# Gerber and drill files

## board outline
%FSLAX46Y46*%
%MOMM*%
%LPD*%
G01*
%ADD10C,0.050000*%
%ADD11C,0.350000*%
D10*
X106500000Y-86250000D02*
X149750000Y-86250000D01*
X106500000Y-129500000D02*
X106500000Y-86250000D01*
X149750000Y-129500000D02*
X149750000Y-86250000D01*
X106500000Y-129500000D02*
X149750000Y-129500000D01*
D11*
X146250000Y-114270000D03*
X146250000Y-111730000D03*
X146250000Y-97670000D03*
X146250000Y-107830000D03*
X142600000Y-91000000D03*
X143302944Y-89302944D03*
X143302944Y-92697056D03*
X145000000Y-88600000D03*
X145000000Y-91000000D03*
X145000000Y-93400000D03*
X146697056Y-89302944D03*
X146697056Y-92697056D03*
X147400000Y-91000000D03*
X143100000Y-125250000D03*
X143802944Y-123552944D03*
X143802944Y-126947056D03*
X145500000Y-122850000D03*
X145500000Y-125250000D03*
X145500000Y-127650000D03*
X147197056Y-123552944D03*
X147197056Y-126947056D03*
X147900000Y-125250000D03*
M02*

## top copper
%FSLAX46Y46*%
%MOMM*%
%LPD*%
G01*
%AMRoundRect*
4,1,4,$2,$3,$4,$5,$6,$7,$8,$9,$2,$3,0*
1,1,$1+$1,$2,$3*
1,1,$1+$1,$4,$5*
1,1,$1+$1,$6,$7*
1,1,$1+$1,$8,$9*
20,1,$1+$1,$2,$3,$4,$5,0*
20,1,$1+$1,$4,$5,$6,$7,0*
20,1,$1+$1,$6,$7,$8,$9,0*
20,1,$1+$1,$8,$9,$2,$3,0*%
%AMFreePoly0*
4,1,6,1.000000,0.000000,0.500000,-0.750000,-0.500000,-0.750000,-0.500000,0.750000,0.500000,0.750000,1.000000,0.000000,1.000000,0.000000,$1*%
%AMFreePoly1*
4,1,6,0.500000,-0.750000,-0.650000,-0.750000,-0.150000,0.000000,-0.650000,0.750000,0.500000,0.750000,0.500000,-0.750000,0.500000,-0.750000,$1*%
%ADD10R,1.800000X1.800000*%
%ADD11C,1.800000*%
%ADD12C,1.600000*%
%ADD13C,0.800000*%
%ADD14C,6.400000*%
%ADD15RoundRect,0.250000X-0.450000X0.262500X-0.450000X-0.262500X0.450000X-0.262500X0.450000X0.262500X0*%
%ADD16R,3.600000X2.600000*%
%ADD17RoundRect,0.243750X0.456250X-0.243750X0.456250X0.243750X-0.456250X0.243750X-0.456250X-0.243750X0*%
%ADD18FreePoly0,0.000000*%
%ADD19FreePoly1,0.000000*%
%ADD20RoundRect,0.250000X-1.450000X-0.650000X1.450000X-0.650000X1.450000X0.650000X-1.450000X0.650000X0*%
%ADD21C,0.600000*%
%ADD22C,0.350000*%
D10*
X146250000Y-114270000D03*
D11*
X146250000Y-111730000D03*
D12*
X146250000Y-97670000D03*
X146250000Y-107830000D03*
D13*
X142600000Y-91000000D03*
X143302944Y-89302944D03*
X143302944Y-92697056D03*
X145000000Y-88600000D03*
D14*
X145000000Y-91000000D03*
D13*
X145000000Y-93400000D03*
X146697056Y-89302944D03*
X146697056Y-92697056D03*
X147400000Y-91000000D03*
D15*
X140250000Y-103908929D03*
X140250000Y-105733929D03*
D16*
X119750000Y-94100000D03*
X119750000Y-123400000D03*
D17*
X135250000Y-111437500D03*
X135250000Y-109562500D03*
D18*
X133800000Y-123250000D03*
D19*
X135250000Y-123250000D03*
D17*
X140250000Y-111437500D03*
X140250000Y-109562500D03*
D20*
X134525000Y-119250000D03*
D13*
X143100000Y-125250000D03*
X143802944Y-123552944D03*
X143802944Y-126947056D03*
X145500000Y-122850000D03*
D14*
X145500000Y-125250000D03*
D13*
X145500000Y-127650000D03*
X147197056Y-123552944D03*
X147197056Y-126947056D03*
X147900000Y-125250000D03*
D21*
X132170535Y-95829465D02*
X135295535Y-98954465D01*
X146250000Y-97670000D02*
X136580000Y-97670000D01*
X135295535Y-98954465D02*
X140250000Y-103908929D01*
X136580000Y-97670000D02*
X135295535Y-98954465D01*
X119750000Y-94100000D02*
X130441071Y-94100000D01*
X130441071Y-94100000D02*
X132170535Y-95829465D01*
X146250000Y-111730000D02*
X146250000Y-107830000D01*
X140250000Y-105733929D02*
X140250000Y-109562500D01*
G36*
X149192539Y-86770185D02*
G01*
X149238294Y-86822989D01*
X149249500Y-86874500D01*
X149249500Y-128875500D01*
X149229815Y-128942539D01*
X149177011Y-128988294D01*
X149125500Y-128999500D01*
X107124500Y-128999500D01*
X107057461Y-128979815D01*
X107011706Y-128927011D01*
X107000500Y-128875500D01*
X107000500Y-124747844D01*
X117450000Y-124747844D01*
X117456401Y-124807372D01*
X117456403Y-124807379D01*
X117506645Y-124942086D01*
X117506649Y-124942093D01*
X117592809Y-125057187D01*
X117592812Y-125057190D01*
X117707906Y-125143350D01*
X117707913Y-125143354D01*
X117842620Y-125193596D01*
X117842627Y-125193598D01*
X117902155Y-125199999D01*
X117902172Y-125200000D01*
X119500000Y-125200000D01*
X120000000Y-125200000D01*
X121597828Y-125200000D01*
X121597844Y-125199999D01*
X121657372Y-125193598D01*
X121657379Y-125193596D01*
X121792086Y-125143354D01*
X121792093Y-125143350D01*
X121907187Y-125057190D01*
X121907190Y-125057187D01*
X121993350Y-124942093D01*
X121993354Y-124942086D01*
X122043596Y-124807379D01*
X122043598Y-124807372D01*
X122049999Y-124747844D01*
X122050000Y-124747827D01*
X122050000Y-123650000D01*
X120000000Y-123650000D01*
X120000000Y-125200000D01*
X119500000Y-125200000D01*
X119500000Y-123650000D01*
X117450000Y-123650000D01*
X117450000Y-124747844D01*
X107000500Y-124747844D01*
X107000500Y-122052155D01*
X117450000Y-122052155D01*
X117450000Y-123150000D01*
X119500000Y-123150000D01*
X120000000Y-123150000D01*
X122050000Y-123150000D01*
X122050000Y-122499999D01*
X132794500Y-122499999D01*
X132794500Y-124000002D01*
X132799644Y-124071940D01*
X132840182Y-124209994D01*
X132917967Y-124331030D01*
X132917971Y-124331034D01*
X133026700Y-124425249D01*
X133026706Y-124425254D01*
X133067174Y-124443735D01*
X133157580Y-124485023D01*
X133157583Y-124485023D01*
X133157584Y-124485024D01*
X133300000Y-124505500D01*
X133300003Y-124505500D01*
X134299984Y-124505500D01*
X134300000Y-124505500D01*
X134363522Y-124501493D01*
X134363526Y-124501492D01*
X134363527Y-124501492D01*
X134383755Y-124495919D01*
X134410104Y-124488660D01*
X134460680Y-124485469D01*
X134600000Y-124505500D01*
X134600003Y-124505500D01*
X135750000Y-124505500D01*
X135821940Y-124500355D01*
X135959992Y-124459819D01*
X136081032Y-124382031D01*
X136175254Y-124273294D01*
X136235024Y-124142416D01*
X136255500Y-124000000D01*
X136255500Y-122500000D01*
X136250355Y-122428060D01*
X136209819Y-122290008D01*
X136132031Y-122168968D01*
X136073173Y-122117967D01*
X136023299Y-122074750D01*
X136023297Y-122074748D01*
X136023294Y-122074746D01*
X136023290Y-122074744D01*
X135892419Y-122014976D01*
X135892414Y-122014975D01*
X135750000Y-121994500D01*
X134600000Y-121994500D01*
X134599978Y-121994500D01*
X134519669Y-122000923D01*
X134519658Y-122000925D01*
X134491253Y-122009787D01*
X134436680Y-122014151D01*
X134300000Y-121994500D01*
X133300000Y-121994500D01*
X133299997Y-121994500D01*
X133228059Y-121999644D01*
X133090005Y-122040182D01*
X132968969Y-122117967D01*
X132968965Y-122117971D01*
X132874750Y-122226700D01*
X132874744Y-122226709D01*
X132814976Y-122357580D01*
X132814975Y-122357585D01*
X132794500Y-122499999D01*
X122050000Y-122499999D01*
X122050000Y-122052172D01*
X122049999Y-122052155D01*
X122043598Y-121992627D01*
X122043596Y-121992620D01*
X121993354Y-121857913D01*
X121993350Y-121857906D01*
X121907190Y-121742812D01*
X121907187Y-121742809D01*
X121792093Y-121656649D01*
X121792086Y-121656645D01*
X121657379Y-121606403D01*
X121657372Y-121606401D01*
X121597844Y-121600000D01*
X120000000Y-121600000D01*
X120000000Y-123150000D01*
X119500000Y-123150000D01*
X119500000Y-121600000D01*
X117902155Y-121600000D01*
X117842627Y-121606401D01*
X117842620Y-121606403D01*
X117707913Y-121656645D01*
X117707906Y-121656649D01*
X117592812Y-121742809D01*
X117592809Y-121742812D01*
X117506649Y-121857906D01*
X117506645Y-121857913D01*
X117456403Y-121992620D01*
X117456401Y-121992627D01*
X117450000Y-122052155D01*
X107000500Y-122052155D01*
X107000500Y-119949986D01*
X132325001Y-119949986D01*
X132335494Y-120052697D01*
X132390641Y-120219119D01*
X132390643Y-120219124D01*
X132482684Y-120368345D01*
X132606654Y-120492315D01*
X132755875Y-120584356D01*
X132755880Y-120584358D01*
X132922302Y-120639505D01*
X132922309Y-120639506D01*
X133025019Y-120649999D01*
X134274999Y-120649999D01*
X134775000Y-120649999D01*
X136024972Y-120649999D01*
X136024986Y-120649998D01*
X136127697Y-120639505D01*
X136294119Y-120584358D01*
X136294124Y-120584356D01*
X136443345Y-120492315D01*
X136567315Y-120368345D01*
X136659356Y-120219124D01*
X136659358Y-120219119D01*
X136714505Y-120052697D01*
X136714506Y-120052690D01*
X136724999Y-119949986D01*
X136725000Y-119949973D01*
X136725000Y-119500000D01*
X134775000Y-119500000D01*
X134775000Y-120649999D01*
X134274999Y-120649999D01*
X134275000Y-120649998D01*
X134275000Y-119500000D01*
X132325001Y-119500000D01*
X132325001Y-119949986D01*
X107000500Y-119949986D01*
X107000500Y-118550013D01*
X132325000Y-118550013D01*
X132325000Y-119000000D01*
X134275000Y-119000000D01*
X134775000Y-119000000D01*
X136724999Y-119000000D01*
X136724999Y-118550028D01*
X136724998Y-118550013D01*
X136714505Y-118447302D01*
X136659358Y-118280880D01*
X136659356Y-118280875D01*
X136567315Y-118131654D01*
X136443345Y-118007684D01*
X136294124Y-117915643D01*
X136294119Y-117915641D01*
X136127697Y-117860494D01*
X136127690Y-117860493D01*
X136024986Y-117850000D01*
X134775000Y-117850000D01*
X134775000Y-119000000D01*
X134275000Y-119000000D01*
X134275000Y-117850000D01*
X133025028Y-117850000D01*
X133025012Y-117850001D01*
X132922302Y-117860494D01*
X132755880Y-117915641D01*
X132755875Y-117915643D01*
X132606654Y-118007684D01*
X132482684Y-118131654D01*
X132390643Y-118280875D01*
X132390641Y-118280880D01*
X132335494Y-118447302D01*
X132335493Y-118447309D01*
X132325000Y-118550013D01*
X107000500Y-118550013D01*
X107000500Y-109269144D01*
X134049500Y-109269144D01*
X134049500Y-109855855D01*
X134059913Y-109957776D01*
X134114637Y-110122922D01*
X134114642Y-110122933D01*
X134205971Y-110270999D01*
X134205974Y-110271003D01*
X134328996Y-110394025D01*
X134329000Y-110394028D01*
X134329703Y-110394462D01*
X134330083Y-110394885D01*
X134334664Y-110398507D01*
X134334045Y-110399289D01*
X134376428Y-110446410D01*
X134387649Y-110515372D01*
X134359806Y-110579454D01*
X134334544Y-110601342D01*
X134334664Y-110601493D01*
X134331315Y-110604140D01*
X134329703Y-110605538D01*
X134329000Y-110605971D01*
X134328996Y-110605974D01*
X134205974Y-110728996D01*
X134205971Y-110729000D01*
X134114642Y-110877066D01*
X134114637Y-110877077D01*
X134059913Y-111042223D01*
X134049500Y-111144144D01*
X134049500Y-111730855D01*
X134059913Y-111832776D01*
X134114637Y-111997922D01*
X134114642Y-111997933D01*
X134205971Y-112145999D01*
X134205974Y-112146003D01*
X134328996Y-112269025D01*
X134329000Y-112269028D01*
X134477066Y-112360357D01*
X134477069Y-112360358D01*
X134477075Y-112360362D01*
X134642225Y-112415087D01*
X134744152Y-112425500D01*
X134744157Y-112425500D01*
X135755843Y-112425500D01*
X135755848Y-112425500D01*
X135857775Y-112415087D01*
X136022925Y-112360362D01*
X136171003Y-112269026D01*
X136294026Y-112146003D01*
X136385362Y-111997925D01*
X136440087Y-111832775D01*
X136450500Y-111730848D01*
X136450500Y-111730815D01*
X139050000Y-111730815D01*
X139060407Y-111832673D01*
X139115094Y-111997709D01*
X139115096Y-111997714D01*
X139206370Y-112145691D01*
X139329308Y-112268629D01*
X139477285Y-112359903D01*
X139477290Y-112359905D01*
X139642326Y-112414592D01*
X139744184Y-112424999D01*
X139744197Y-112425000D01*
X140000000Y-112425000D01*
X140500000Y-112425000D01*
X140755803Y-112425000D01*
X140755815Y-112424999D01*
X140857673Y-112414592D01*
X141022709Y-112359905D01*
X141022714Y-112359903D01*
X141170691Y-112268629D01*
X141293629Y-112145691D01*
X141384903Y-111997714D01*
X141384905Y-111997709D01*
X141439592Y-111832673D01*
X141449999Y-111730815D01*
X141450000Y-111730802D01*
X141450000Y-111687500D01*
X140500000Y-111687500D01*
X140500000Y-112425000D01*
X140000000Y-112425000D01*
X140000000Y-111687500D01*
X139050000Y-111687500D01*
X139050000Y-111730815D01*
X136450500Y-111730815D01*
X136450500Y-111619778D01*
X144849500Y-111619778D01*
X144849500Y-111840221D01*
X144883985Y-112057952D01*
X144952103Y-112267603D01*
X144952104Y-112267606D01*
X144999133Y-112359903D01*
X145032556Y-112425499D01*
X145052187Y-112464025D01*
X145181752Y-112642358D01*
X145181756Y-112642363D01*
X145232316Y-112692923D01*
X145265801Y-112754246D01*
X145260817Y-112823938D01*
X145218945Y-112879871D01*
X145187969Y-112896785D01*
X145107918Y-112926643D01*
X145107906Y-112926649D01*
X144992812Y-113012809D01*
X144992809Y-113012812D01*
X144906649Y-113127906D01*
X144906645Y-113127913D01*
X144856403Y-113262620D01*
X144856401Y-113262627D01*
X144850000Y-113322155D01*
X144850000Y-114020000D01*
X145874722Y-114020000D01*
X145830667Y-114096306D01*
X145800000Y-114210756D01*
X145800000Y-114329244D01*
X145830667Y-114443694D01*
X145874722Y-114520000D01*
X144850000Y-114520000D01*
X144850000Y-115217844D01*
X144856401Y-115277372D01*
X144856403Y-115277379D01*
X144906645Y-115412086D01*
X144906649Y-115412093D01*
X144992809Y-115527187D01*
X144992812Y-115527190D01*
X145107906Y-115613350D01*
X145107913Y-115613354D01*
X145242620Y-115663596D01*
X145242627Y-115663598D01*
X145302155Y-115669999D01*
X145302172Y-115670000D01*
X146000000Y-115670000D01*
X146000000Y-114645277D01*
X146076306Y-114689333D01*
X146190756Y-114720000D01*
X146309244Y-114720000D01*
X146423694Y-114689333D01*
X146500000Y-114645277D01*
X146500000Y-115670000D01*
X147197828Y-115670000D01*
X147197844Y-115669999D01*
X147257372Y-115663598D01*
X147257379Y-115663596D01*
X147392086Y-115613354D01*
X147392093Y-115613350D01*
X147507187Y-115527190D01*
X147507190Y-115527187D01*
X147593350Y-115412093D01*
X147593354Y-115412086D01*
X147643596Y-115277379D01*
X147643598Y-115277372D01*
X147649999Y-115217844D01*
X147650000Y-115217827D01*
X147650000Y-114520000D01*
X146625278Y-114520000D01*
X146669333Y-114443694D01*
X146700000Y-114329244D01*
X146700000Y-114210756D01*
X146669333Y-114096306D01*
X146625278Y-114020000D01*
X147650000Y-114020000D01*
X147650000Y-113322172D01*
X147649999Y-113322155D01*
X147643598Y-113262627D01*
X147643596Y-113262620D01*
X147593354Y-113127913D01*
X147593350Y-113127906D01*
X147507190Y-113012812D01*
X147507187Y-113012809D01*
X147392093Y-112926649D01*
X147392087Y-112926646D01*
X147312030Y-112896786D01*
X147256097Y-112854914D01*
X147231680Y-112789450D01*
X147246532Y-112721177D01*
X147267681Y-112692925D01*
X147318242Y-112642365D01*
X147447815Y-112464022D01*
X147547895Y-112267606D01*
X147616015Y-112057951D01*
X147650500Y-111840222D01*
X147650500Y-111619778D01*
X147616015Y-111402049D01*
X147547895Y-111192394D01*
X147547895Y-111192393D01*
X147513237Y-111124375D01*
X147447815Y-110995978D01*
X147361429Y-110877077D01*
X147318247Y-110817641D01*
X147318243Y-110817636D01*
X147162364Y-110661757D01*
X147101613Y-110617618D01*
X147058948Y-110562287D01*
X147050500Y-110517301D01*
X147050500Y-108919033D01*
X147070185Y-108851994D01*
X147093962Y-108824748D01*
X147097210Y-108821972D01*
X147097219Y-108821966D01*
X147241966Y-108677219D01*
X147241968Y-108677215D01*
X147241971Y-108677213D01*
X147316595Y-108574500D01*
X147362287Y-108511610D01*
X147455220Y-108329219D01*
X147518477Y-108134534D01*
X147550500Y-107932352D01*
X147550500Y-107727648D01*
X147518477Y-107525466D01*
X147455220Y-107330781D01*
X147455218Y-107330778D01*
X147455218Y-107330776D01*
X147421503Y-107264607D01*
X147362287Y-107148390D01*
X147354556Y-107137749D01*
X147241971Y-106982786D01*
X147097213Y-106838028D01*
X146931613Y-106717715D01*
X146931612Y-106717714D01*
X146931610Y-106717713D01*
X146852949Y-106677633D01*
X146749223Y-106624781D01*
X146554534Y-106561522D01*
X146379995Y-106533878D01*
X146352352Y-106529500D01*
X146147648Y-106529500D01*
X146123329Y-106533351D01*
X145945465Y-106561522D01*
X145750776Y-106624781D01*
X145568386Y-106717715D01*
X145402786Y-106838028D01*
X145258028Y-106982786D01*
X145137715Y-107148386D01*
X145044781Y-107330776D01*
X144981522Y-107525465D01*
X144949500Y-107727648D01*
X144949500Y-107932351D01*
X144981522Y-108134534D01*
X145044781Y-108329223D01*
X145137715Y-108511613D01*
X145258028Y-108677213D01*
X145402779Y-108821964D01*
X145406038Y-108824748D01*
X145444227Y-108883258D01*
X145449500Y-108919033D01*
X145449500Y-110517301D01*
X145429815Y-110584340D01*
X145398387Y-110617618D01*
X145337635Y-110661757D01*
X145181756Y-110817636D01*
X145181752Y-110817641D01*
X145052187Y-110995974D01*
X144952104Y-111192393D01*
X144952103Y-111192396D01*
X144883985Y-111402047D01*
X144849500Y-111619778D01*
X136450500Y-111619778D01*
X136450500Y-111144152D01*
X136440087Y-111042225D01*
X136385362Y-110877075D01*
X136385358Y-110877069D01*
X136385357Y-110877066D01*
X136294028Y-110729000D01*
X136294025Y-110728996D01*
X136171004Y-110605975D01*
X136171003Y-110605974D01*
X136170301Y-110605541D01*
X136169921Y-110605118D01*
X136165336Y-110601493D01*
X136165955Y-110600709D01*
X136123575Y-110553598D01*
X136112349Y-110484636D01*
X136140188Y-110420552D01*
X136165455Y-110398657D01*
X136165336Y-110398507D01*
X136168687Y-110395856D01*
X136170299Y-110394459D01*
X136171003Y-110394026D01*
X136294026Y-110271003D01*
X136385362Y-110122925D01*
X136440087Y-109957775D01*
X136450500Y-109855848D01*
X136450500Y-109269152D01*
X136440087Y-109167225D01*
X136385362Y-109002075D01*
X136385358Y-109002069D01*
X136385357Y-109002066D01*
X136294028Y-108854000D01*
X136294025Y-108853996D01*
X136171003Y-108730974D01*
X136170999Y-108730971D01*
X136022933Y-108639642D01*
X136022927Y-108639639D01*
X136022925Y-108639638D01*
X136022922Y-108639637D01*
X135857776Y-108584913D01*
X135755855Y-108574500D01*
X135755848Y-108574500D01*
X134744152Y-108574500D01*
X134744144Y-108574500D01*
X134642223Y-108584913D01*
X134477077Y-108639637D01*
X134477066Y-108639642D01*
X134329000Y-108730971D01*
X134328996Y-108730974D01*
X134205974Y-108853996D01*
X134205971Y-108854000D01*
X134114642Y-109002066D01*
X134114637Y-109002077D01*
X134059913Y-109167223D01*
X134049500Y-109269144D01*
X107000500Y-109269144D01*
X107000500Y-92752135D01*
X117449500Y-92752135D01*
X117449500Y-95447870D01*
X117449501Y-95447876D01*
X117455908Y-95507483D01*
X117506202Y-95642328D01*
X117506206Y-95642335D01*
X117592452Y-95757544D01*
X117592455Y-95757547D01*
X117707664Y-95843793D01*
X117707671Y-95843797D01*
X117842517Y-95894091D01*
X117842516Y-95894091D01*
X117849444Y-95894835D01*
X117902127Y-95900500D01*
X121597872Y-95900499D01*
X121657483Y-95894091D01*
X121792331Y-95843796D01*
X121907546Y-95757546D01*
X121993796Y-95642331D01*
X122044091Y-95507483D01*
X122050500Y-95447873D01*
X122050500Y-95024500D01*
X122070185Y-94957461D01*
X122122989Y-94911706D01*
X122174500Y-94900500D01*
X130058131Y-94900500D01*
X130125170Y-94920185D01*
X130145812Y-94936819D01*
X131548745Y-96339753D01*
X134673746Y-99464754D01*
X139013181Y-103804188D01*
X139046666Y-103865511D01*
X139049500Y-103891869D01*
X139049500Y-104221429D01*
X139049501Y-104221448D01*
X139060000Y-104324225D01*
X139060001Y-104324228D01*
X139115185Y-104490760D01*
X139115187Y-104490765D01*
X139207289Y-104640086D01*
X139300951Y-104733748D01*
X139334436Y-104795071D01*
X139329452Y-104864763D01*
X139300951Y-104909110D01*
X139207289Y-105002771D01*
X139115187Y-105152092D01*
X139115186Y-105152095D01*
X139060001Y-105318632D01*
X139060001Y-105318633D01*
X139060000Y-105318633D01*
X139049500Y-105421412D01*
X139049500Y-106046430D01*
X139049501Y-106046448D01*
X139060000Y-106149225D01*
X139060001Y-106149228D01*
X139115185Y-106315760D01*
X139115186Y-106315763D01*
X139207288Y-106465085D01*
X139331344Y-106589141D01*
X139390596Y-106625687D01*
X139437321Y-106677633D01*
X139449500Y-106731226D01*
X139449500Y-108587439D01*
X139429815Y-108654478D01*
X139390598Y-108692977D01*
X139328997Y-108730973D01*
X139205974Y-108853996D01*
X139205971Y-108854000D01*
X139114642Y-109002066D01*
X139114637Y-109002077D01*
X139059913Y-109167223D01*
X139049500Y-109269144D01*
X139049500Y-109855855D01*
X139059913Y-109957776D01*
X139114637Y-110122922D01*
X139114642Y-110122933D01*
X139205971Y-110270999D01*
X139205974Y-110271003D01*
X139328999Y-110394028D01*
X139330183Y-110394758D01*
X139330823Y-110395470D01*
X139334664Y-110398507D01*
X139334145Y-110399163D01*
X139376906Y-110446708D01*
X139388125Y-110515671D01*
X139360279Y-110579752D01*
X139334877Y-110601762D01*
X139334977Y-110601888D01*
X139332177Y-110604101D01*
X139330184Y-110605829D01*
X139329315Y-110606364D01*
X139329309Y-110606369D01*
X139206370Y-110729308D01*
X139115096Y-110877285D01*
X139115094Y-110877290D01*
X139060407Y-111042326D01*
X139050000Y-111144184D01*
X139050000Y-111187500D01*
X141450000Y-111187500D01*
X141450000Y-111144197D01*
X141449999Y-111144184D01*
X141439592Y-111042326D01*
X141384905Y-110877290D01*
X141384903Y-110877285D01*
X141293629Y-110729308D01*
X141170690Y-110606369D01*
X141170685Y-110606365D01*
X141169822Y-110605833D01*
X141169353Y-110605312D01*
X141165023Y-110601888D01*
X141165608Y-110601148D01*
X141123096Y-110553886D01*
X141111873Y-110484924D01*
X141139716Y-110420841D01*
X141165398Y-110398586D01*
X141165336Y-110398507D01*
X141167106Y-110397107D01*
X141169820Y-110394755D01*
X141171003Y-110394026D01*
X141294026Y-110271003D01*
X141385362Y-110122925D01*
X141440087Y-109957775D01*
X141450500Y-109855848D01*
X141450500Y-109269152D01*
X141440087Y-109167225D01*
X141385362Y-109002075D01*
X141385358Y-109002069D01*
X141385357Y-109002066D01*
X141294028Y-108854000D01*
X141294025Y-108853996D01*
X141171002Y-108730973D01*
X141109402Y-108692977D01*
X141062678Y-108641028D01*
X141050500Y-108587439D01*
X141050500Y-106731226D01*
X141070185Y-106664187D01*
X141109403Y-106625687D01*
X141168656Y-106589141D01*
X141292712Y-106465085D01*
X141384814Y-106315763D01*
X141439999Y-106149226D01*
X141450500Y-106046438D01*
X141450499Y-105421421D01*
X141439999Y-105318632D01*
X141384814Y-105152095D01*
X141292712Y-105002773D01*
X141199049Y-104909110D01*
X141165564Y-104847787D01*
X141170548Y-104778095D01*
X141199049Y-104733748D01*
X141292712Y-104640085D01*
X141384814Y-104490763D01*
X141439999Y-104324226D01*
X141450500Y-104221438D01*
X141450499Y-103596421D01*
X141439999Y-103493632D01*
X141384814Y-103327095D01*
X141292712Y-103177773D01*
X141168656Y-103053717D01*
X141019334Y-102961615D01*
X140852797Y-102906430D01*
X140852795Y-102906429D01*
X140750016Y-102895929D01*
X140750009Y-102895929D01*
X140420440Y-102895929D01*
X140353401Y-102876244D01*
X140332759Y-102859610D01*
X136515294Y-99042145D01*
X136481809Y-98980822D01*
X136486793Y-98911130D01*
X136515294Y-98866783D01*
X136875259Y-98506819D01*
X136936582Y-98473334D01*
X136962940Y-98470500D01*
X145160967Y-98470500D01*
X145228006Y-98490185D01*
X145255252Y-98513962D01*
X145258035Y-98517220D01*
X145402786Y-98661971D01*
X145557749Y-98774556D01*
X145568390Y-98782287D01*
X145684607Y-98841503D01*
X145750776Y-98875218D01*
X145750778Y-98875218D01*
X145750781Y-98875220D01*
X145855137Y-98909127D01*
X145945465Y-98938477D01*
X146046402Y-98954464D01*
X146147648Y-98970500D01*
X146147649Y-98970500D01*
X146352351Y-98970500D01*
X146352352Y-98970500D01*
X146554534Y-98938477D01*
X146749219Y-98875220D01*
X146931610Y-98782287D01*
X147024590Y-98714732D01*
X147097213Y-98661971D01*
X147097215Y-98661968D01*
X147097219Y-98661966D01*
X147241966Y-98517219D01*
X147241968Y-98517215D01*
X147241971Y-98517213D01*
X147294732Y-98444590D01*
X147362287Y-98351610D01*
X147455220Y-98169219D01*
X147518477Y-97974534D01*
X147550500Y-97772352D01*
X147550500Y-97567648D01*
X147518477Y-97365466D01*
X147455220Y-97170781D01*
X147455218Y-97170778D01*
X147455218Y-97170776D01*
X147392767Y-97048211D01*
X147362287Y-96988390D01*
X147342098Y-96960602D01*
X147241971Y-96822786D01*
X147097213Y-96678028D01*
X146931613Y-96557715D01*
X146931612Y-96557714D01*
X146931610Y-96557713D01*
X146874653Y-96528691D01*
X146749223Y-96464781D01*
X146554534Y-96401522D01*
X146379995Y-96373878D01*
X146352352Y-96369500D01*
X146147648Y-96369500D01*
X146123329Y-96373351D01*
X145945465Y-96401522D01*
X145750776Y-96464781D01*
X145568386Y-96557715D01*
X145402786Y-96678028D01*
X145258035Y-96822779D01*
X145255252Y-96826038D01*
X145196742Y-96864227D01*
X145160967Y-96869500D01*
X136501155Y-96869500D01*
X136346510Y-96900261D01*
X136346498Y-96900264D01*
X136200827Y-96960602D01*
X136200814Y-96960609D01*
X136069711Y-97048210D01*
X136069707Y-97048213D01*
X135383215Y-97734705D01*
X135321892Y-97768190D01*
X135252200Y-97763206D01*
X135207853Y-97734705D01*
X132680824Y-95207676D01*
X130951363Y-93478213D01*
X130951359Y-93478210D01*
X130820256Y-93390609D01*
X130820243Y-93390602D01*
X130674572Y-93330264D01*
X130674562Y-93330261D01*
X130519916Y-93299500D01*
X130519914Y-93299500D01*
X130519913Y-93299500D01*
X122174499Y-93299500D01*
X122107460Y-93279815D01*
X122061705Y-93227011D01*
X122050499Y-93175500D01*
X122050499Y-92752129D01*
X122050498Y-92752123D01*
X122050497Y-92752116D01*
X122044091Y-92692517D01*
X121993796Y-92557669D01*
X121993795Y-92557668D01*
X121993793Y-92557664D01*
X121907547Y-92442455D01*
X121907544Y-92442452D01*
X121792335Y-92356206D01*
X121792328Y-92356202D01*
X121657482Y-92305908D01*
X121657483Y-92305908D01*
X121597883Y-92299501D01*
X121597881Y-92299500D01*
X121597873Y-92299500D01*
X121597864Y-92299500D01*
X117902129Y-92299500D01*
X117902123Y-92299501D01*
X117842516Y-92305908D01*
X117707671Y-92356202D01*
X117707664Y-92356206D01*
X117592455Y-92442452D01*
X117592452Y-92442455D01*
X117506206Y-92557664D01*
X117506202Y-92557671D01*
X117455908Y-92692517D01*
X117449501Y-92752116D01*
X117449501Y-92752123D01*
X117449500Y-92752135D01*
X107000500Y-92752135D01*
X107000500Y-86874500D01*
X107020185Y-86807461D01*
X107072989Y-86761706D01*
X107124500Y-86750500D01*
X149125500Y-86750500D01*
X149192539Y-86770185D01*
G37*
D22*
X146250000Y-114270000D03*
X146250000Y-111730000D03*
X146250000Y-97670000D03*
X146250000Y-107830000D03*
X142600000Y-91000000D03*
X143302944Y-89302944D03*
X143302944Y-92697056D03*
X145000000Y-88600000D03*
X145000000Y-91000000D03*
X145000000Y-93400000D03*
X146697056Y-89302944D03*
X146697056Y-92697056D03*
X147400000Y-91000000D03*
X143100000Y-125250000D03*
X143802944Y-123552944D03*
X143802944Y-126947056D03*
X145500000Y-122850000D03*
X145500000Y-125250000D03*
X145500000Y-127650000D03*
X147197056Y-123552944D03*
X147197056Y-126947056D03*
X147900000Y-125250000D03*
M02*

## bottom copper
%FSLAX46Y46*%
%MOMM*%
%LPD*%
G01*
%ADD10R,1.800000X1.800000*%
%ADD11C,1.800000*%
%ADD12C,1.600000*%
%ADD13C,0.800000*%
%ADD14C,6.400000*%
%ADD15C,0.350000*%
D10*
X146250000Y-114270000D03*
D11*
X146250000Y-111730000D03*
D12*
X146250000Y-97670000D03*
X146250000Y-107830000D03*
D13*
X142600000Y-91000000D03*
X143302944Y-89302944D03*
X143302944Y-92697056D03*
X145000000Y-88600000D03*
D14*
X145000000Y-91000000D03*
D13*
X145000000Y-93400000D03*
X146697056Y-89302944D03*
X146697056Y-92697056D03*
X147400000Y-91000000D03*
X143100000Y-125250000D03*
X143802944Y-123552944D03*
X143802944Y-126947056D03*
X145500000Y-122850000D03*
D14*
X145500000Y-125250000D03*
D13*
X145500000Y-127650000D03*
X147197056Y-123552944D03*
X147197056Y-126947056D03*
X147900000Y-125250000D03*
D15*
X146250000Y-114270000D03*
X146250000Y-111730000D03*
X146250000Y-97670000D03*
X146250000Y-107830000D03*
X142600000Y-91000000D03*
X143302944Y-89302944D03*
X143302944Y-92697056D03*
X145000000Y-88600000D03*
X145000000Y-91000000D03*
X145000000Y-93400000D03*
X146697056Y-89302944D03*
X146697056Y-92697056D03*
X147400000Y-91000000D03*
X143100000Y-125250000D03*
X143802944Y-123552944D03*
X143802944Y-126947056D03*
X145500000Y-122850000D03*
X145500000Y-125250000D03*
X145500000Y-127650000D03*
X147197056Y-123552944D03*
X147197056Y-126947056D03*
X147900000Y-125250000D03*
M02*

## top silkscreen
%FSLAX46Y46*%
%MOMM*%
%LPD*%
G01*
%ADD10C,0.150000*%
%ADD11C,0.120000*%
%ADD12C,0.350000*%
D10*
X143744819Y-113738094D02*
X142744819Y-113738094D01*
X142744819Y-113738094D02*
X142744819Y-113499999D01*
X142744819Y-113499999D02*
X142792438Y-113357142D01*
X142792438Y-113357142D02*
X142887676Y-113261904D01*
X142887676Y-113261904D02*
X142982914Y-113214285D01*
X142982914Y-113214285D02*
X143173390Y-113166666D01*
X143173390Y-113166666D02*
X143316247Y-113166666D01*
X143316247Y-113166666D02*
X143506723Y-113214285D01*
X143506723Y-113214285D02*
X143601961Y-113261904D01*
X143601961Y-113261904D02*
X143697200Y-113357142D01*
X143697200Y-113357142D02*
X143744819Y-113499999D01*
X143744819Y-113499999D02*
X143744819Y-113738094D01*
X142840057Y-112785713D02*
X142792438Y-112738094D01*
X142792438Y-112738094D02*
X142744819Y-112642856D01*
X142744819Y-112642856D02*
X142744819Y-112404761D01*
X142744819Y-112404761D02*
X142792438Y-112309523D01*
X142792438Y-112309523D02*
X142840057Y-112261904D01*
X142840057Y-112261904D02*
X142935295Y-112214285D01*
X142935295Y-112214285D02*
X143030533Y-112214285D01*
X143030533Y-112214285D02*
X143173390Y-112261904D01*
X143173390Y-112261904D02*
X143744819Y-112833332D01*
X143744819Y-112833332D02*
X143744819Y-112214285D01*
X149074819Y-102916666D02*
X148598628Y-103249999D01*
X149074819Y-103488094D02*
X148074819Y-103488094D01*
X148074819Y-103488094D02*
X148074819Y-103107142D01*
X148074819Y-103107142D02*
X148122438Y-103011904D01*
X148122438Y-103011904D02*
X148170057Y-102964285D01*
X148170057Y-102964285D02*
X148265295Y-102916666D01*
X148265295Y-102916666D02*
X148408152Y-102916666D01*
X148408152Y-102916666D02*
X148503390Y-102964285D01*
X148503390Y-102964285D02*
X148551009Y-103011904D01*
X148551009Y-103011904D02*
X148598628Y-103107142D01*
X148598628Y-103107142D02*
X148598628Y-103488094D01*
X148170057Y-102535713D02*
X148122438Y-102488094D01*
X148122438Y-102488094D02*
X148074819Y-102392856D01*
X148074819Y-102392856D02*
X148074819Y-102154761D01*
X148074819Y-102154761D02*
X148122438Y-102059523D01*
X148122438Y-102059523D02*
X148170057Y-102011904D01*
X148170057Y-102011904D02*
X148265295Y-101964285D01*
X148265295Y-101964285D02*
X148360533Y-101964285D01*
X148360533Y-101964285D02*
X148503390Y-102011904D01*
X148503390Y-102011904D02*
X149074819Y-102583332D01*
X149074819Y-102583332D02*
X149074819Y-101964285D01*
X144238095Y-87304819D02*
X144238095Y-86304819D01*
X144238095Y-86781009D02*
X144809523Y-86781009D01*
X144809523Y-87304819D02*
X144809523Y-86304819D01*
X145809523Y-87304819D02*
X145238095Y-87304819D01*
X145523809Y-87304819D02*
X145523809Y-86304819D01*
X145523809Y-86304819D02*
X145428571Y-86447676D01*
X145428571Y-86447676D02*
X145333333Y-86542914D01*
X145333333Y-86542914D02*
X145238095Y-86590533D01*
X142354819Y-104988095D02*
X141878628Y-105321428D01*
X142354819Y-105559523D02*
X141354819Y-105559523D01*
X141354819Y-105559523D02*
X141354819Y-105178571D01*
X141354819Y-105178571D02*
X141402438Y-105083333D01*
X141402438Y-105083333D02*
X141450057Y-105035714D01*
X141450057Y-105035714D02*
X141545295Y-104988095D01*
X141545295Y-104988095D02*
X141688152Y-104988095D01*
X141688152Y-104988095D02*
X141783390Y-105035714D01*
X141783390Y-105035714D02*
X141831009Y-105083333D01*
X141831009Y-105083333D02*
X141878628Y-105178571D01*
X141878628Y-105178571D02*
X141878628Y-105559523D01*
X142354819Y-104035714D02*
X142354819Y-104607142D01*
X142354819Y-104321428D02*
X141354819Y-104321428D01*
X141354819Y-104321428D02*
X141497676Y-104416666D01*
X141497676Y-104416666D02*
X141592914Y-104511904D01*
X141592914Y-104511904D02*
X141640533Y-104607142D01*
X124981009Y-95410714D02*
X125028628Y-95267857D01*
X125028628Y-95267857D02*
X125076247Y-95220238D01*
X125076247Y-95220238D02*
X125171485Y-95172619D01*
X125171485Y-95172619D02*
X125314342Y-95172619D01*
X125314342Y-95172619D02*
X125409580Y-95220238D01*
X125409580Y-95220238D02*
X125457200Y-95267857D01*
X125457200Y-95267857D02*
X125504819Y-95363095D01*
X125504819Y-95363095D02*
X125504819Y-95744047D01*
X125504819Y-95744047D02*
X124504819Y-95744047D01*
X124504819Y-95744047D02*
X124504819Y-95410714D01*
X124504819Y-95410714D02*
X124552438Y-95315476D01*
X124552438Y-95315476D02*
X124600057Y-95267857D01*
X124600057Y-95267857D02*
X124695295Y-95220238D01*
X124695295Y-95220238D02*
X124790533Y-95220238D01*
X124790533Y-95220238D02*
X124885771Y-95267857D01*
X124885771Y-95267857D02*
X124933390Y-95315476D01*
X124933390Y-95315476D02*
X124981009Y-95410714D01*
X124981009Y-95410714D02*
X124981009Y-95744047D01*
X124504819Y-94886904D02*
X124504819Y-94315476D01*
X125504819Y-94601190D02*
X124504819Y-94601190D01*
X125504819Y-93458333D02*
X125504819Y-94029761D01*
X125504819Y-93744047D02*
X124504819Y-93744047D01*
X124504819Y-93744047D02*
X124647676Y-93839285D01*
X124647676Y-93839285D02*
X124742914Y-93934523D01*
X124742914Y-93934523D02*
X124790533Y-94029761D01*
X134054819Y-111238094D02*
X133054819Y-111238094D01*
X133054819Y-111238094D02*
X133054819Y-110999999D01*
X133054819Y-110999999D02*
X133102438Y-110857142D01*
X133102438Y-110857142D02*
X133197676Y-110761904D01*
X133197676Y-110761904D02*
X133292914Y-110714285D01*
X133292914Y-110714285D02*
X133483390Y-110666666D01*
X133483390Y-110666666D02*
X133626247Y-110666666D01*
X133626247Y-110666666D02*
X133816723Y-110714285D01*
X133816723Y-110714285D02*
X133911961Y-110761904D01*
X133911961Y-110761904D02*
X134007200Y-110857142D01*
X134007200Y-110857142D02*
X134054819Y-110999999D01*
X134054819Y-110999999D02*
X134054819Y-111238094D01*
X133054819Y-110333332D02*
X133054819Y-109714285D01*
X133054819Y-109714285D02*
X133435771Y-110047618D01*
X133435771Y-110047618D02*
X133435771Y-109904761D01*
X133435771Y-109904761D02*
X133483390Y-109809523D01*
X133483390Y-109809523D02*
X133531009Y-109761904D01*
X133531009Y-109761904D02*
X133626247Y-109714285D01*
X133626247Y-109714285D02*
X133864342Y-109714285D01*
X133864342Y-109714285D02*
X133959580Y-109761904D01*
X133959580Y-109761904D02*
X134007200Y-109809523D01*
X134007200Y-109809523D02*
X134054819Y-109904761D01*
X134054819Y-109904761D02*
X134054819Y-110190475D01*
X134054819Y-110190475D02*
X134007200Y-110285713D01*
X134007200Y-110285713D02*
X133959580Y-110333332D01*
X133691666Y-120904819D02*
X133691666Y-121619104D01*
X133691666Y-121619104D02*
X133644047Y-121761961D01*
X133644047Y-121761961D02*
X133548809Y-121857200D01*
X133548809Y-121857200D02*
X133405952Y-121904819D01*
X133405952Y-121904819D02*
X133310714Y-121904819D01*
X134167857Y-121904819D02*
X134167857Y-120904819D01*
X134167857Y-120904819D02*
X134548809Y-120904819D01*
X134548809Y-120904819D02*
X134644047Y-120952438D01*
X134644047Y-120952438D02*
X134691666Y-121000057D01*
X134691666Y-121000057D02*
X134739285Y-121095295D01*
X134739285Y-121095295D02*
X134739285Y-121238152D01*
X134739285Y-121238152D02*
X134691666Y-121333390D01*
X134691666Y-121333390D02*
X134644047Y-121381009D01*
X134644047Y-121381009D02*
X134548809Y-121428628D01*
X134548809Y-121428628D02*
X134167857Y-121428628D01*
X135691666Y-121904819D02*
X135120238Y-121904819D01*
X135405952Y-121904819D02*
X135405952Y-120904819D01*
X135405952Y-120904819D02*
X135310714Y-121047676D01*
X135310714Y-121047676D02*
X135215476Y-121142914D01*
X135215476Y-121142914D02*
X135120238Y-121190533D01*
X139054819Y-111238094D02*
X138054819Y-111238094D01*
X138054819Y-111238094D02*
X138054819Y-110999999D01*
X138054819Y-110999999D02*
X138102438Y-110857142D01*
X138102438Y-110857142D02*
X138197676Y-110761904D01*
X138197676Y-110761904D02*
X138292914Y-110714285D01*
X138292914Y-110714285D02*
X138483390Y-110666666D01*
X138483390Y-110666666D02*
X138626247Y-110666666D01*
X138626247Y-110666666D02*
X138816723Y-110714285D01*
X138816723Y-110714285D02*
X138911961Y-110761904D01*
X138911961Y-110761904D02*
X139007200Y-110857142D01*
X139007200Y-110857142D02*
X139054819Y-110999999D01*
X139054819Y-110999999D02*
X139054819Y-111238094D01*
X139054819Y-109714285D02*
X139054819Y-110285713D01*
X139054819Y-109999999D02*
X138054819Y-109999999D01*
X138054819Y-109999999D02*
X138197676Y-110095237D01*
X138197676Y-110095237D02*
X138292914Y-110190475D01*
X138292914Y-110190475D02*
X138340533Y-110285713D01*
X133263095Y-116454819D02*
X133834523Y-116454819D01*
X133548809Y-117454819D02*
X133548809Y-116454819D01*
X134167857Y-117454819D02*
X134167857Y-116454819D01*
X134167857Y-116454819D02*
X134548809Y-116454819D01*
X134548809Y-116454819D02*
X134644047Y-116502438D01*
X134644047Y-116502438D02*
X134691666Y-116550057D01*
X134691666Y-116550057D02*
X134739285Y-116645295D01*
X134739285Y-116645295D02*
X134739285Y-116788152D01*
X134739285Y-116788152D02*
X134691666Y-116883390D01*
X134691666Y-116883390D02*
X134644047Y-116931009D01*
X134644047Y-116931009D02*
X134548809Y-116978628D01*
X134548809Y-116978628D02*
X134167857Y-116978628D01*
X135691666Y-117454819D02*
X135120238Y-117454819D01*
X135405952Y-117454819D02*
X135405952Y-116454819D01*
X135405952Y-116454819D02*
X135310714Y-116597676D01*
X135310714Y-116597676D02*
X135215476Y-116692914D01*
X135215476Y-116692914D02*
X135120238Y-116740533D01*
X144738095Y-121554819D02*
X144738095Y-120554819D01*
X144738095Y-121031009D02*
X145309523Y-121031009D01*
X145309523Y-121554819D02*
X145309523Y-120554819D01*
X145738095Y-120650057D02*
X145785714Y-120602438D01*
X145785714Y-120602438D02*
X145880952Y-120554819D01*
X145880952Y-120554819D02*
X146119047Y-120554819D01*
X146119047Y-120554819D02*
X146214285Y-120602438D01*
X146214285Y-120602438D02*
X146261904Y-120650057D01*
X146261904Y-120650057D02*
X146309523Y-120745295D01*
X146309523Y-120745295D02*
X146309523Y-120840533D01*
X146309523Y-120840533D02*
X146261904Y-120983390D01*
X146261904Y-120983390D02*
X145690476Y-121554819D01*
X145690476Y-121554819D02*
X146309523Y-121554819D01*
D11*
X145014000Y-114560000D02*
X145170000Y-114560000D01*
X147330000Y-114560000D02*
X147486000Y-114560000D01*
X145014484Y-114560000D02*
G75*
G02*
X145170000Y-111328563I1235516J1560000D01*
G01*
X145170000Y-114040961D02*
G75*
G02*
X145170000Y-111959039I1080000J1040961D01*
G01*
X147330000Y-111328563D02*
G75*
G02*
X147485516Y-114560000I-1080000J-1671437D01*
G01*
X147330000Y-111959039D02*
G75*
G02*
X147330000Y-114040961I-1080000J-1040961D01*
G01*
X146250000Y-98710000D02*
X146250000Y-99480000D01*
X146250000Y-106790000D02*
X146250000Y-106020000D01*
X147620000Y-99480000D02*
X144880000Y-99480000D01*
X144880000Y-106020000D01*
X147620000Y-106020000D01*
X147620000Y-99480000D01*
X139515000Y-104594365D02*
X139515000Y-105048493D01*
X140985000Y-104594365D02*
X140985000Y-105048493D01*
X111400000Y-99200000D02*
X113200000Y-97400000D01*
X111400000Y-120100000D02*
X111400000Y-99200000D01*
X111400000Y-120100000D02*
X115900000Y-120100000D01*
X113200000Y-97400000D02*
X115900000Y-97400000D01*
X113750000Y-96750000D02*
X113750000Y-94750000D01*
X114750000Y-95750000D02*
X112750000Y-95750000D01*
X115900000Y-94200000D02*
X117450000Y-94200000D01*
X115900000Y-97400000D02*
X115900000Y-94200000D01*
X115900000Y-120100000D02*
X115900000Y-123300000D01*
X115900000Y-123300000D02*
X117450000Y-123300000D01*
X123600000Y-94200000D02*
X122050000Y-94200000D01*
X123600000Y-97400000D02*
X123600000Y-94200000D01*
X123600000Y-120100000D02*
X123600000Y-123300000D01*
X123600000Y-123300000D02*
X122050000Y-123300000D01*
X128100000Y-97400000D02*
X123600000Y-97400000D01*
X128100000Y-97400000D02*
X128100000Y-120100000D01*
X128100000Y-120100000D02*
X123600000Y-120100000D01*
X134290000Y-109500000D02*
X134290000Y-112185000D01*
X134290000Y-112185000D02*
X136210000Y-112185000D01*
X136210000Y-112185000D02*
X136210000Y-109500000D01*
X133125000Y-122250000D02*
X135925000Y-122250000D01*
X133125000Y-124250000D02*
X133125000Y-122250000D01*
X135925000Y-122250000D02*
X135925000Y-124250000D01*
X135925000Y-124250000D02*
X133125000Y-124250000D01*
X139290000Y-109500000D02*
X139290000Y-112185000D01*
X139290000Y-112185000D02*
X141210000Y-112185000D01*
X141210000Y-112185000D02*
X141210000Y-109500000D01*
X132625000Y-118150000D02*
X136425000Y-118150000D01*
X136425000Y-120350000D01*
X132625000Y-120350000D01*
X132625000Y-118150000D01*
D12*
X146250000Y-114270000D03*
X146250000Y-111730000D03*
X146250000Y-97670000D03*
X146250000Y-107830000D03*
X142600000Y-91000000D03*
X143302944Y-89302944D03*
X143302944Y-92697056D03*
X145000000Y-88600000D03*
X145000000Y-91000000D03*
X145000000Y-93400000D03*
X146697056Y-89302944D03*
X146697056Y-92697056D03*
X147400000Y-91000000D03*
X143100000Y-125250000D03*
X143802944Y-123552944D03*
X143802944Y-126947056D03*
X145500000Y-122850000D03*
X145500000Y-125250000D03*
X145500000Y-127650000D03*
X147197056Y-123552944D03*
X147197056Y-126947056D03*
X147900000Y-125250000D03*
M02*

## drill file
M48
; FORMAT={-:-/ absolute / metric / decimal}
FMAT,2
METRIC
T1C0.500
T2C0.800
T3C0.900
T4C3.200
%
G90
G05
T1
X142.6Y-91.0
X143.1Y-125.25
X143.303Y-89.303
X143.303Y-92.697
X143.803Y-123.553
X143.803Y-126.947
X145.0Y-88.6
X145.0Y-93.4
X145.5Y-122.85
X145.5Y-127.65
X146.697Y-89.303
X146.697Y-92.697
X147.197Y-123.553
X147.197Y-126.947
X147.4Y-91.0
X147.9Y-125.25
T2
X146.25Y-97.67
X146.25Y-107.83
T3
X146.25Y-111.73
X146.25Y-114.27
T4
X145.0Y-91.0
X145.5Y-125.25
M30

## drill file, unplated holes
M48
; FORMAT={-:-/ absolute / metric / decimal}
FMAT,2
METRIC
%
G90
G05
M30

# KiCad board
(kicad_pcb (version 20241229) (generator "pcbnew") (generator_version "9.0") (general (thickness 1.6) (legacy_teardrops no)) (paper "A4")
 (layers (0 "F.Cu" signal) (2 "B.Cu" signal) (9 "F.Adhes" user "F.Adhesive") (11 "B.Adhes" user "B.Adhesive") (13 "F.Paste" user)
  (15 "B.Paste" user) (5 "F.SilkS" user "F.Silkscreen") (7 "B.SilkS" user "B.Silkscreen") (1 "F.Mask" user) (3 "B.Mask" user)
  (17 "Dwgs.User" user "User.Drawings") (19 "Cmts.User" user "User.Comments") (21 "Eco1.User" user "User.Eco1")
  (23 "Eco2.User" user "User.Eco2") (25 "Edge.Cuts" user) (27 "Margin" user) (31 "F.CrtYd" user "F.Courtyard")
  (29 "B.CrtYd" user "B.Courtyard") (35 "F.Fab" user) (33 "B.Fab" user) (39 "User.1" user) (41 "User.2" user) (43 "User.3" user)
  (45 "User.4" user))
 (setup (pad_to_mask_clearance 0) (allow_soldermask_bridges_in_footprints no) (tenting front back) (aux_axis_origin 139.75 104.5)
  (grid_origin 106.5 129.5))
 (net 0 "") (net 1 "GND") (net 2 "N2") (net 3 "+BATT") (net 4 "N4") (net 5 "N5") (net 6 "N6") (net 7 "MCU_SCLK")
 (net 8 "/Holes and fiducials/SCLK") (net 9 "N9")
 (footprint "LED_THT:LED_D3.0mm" (layer "F.Cu") (at 146.25 114.27 90)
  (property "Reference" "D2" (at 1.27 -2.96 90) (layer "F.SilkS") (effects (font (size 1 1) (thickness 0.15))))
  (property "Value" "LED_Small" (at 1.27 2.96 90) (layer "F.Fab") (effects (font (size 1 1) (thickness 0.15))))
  (fp_line (start -0.29 -1.236) (end -0.29 -1.08) (stroke (width 0.12) (type solid)) (layer "F.SilkS"))
  (fp_line (start -0.29 1.08) (end -0.29 1.236) (stroke (width 0.12) (type solid)) (layer "F.SilkS"))
  (fp_arc (start -0.29 -1.235516) (mid 1.36566 -1.987699) (end 2.941437 -1.08) (stroke (width 0.12) (type solid)) (layer "F.SilkS"))
  (fp_arc (start 0.229039 -1.08) (mid 1.27 -1.5) (end 2.310961 -1.08) (stroke (width 0.12) (type solid)) (layer "F.SilkS"))
  (fp_arc (start 2.941437 1.08) (mid 1.36566 1.987699) (end -0.29 1.235516) (stroke (width 0.12) (type solid)) (layer "F.SilkS"))
  (fp_arc (start 2.310961 1.08) (mid 1.27 1.5) (end 0.229039 1.08) (stroke (width 0.12) (type solid)) (layer "F.SilkS"))
  (pad "1" thru_hole rect (at 0 0 90) (size 1.8 1.8) (drill 0.9) (layers "*.Cu" "*.Mask") (remove_unused_layers no) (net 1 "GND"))
  (pad "2" thru_hole circle (at 2.54 0 90) (size 1.8 1.8) (drill 0.9) (layers "*.Cu" "*.Mask") (remove_unused_layers no) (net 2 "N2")))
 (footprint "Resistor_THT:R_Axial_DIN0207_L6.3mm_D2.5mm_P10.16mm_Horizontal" (layer "F.Cu") (at 146.25 97.67 -90)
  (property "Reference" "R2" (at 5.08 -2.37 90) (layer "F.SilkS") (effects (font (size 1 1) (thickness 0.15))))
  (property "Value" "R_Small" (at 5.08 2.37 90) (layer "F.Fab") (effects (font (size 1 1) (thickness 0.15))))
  (fp_line (start 1.04 0) (end 1.81 0) (stroke (width 0.12) (type solid)) (layer "F.SilkS"))
  (fp_line (start 9.12 0) (end 8.35 0) (stroke (width 0.12) (type solid)) (layer "F.SilkS"))
  (fp_rect (start 1.81 -1.37) (end 8.35 1.37) (stroke (width 0.12) (type solid)) (fill no) (layer "F.SilkS"))
  (pad "1" thru_hole circle (at 0 0 270) (size 1.6 1.6) (drill 0.8) (layers "*.Cu" "*.Mask") (remove_unused_layers no) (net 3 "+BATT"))
  (pad "2" thru_hole circle (at 10.16 0 270) (size 1.6 1.6) (drill 0.8) (layers "*.Cu" "*.Mask") (remove_unused_layers no) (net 2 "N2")))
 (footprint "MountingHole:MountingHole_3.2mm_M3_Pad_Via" (layer "F.Cu") (at 145 91)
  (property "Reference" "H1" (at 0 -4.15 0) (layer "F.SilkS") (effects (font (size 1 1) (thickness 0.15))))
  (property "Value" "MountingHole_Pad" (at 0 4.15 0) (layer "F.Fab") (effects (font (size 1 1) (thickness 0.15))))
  (pad "1" thru_hole circle (at -2.4 0) (size 0.8 0.8) (drill 0.5) (layers "*.Cu" "*.Mask") (remove_unused_layers no) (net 1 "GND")
   (zone_connect 2))
  (pad "1" thru_hole circle (at -1.697056 -1.697056) (size 0.8 0.8) (drill 0.5) (layers "*.Cu" "*.Mask") (remove_unused_layers no)
   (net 1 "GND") (zone_connect 2))
  (pad "1" thru_hole circle (at -1.697056 1.697056) (size 0.8 0.8) (drill 0.5) (layers "*.Cu" "*.Mask") (remove_unused_layers no)
   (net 1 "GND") (zone_connect 2))
  (pad "1" thru_hole circle (at 0 -2.4) (size 0.8 0.8) (drill 0.5) (layers "*.Cu" "*.Mask") (remove_unused_layers no) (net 1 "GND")
   (zone_connect 2))
  (pad "1" thru_hole circle (at 0 0) (size 6.4 6.4) (drill 3.2) (layers "*.Cu" "*.Mask") (remove_unused_layers no) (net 1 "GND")
   (zone_connect 2))
  (pad "1" thru_hole circle (at 0 2.4) (size 0.8 0.8) (drill 0.5) (layers "*.Cu" "*.Mask") (remove_unused_layers no) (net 1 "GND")
   (zone_connect 2))
  (pad "1" thru_hole circle (at 1.697056 -1.697056) (size 0.8 0.8) (drill 0.5) (layers "*.Cu" "*.Mask") (remove_unused_layers no)
   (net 1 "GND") (zone_connect 2))
  (pad "1" thru_hole circle (at 1.697056 1.697056) (size 0.8 0.8) (drill 0.5) (layers "*.Cu" "*.Mask") (remove_unused_layers no)
   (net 1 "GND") (zone_connect 2))
  (pad "1" thru_hole circle (at 2.4 0) (size 0.8 0.8) (drill 0.5) (layers "*.Cu" "*.Mask") (remove_unused_layers no) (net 1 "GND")
   (zone_connect 2)))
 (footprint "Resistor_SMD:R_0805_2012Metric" (layer "F.Cu") (at 140.25 104.821429 -90)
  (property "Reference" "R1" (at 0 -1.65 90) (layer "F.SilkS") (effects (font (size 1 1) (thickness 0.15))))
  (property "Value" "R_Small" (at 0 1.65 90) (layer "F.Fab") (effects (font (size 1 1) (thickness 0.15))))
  (fp_line (start -0.227064 0.735) (end 0.227064 0.735) (stroke (width 0.12) (type solid)) (layer "F.SilkS"))
  (fp_line (start -0.227064 -0.735) (end 0.227064 -0.735) (stroke (width 0.12) (type solid)) (layer "F.SilkS"))
  (pad "1" smd roundrect (at -0.9125 0 270) (size 1.025 1.4) (layers "F.Cu" "F.Mask" "F.Paste") (roundrect_rratio 0.243902) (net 3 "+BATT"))
  (pad "2" smd roundrect (at 0.9125 0 270) (size 1.025 1.4) (layers "F.Cu" "F.Mask" "F.Paste") (roundrect_rratio 0.243902) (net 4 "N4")))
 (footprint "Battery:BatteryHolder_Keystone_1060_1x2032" (layer "F.Cu") (at 119.75 108.75 -90)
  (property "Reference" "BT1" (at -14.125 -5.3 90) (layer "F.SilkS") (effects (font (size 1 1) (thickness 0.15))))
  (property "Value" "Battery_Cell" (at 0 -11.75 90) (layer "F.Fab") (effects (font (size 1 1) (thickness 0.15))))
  (fp_line (start -9.55 8.35) (end -11.35 6.55) (stroke (width 0.12) (type solid)) (layer "F.SilkS"))
  (fp_line (start 11.35 8.35) (end -9.55 8.35) (stroke (width 0.12) (type solid)) (layer "F.SilkS"))
  (fp_line (start 11.35 8.35) (end 11.35 3.85) (stroke (width 0.12) (type solid)) (layer "F.SilkS"))
  (fp_line (start -11.35 6.55) (end -11.35 3.85) (stroke (width 0.12) (type solid)) (layer "F.SilkS"))
  (fp_line (start -12 6) (end -14 6) (stroke (width 0.12) (type solid)) (layer "F.SilkS"))
  (fp_line (start -13 5) (end -13 7) (stroke (width 0.12) (type solid)) (layer "F.SilkS"))
  (fp_line (start -14.55 3.85) (end -14.55 2.3) (stroke (width 0.12) (type solid)) (layer "F.SilkS"))
  (fp_line (start -11.35 3.85) (end -14.55 3.85) (stroke (width 0.12) (type solid)) (layer "F.SilkS"))
  (fp_line (start 11.35 3.85) (end 14.55 3.85) (stroke (width 0.12) (type solid)) (layer "F.SilkS"))
  (fp_line (start 14.55 3.85) (end 14.55 2.3) (stroke (width 0.12) (type solid)) (layer "F.SilkS"))
  (fp_line (start -14.55 -3.85) (end -14.55 -2.3) (stroke (width 0.12) (type solid)) (layer "F.SilkS"))
  (fp_line (start -11.35 -3.85) (end -14.55 -3.85) (stroke (width 0.12) (type solid)) (layer "F.SilkS"))
  (fp_line (start 11.35 -3.85) (end 14.55 -3.85) (stroke (width 0.12) (type solid)) (layer "F.SilkS"))
  (fp_line (start 14.55 -3.85) (end 14.55 -2.3) (stroke (width 0.12) (type solid)) (layer "F.SilkS"))
  (fp_line (start -11.35 -8.35) (end -11.35 -3.85) (stroke (width 0.12) (type solid)) (layer "F.SilkS"))
  (fp_line (start -11.35 -8.35) (end 11.35 -8.35) (stroke (width 0.12) (type solid)) (layer "F.SilkS"))
  (fp_line (start 11.35 -8.35) (end 11.35 -3.85) (stroke (width 0.12) (type solid)) (layer "F.SilkS"))
  (pad "1" smd rect (at -14.65 0 90) (size 2.6 3.6) (layers "F.Cu" "F.Mask" "F.Paste") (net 3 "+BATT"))
  (pad "2" smd rect (at 14.65 0 90) (size 2.6 3.6) (layers "F.Cu" "F.Mask" "F.Paste") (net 1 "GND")))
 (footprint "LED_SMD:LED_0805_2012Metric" (layer "F.Cu") (at 135.25 110.5 90)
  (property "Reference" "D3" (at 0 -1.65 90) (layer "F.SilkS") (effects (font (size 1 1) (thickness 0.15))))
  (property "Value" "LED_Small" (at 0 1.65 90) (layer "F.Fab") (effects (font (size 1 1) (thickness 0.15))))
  (fp_line (start 1 -0.96) (end -1.685 -0.96) (stroke (width 0.12) (type solid)) (layer "F.SilkS"))
  (fp_line (start -1.685 -0.96) (end -1.685 0.96) (stroke (width 0.12) (type solid)) (layer "F.SilkS"))
  (fp_line (start -1.685 0.96) (end 1 0.96) (stroke (width 0.12) (type solid)) (layer "F.SilkS"))
  (pad "1" smd roundrect (at -0.9375 0 90) (size 0.975 1.4) (layers "F.Cu" "F.Mask" "F.Paste") (roundrect_rratio 0.25) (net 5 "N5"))
  (pad "2" smd roundrect (at 0.9375 0 90) (size 0.975 1.4) (layers "F.Cu" "F.Mask" "F.Paste") (roundrect_rratio 0.25) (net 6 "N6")))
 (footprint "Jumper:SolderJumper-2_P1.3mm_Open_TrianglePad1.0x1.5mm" (layer "F.Cu") (at 134.525 123.25)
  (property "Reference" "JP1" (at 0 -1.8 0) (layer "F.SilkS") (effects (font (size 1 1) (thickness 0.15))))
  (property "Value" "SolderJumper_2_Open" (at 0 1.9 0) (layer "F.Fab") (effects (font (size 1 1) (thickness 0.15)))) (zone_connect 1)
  (fp_line (start -1.4 -1) (end 1.4 -1) (stroke (width 0.12) (type solid)) (layer "F.SilkS"))
  (fp_line (start -1.4 1) (end -1.4 -1) (stroke (width 0.12) (type solid)) (layer "F.SilkS"))
  (fp_line (start 1.4 -1) (end 1.4 1) (stroke (width 0.12) (type solid)) (layer "F.SilkS"))
  (fp_line (start 1.4 1) (end -1.4 1) (stroke (width 0.12) (type solid)) (layer "F.SilkS"))
  (pad "1" smd custom (at -0.725 0) (size 0.3 0.3) (layers "F.Cu" "F.Mask") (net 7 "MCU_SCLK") (zone_connect 2) (thermal_bridge_angle 45)
   (options (clearance outline) (anchor rect)) (primitives))
  (pad "2" smd custom (at 0.725 0) (size 0.3 0.3) (layers "F.Cu" "F.Mask") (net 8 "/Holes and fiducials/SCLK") (zone_connect 2)
   (thermal_bridge_angle 45) (options (clearance outline) (anchor rect)) (primitives)))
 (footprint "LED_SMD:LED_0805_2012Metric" (layer "F.Cu") (at 140.25 110.5 90)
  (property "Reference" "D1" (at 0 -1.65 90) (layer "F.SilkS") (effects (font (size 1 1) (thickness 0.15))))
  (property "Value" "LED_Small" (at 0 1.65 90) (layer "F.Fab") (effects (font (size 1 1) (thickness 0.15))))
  (fp_line (start 1 -0.96) (end -1.685 -0.96) (stroke (width 0.12) (type solid)) (layer "F.SilkS"))
  (fp_line (start -1.685 -0.96) (end -1.685 0.96) (stroke (width 0.12) (type solid)) (layer "F.SilkS"))
  (fp_line (start -1.685 0.96) (end 1 0.96) (stroke (width 0.12) (type solid)) (layer "F.SilkS"))
  (pad "1" smd roundrect (at -0.9375 0 90) (size 0.975 1.4) (layers "F.Cu" "F.Mask" "F.Paste") (roundrect_rratio 0.25) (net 1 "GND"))
  (pad "2" smd roundrect (at 0.9375 0 90) (size 0.975 1.4) (layers "F.Cu" "F.Mask" "F.Paste") (roundrect_rratio 0.25) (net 4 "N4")))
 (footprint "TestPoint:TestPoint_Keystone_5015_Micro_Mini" (layer "F.Cu") (at 134.525 119.25)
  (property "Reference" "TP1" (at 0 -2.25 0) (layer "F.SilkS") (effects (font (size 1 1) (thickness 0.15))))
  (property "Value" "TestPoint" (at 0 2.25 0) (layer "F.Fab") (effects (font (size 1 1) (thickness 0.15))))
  (fp_rect (start -1.9 -1.1) (end 1.9 1.1) (stroke (width 0.12) (type default)) (fill no) (layer "F.SilkS"))
  (pad "1" smd roundrect (at 0 0) (size 3.4 1.8) (layers "F.Cu" "F.Mask" "F.Paste") (roundrect_rratio 0.1388888889) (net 1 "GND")))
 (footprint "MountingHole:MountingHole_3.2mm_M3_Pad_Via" (layer "F.Cu") (at 145.5 125.25)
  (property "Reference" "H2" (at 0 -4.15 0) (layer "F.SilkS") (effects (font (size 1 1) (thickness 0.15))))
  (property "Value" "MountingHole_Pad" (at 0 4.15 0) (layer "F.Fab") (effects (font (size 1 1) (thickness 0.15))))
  (pad "1" thru_hole circle (at -2.4 0) (size 0.8 0.8) (drill 0.5) (layers "*.Cu" "*.Mask") (remove_unused_layers no) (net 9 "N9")
   (zone_connect 2))
  (pad "1" thru_hole circle (at -1.697056 -1.697056) (size 0.8 0.8) (drill 0.5) (layers "*.Cu" "*.Mask") (remove_unused_layers no)
   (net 9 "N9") (zone_connect 2))
  (pad "1" thru_hole circle (at -1.697056 1.697056) (size 0.8 0.8) (drill 0.5) (layers "*.Cu" "*.Mask") (remove_unused_layers no)
   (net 9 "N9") (zone_connect 2))
  (pad "1" thru_hole circle (at 0 -2.4) (size 0.8 0.8) (drill 0.5) (layers "*.Cu" "*.Mask") (remove_unused_layers no) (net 9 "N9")
   (zone_connect 2))
  (pad "1" thru_hole circle (at 0 0) (size 6.4 6.4) (drill 3.2) (layers "*.Cu" "*.Mask") (remove_unused_layers no) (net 9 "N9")
   (zone_connect 2))
  (pad "1" thru_hole circle (at 0 2.4) (size 0.8 0.8) (drill 0.5) (layers "*.Cu" "*.Mask") (remove_unused_layers no) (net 9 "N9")
   (zone_connect 2))
  (pad "1" thru_hole circle (at 1.697056 -1.697056) (size 0.8 0.8) (drill 0.5) (layers "*.Cu" "*.Mask") (remove_unused_layers no)
   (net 9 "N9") (zone_connect 2))
  (pad "1" thru_hole circle (at 1.697056 1.697056) (size 0.8 0.8) (drill 0.5) (layers "*.Cu" "*.Mask") (remove_unused_layers no)
   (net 9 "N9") (zone_connect 2))
  (pad "1" thru_hole circle (at 2.4 0) (size 0.8 0.8) (drill 0.5) (layers "*.Cu" "*.Mask") (remove_unused_layers no) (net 9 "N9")
   (zone_connect 2)))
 (gr_line (start 106.5 86.25) (end 149.75 86.25) (stroke (width 0.05) (type default)) (layer "Edge.Cuts"))
 (gr_line (start 106.5 129.5) (end 106.5 86.25) (stroke (width 0.05) (type default)) (layer "Edge.Cuts"))
 (gr_line (start 149.75 129.5) (end 149.75 86.25) (stroke (width 0.05) (type default)) (layer "Edge.Cuts"))
 (gr_line (start 106.5 129.5) (end 149.75 129.5) (stroke (width 0.05) (type default)) (layer "Edge.Cuts"))
 (segment (start 132.170535 95.829465) (end 135.295535 98.954465) (width 0.6) (layer "F.Cu") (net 3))
 (segment (start 146.25 97.67) (end 136.58 97.67) (width 0.6) (layer "F.Cu") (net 3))
 (segment (start 135.295535 98.954465) (end 140.25 103.908929) (width 0.6) (layer "F.Cu") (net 3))
 (segment (start 136.58 97.67) (end 135.295535 98.954465) (width 0.6) (layer "F.Cu") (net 3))
 (segment (start 119.75 94.1) (end 130.441071 94.1) (width 0.6) (layer "F.Cu") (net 3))
 (segment (start 130.441071 94.1) (end 132.170535 95.829465) (width 0.6) (layer "F.Cu") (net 3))
 (segment (start 146.25 111.73) (end 146.25 107.83) (width 0.6) (layer "F.Cu") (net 2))
 (segment (start 140.25 105.733929) (end 140.25 109.5625) (width 0.6) (layer "F.Cu") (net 4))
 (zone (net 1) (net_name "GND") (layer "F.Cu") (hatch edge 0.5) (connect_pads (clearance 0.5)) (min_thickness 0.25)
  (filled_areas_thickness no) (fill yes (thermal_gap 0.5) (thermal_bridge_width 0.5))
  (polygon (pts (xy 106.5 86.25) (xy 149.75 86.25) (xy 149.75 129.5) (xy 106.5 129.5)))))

